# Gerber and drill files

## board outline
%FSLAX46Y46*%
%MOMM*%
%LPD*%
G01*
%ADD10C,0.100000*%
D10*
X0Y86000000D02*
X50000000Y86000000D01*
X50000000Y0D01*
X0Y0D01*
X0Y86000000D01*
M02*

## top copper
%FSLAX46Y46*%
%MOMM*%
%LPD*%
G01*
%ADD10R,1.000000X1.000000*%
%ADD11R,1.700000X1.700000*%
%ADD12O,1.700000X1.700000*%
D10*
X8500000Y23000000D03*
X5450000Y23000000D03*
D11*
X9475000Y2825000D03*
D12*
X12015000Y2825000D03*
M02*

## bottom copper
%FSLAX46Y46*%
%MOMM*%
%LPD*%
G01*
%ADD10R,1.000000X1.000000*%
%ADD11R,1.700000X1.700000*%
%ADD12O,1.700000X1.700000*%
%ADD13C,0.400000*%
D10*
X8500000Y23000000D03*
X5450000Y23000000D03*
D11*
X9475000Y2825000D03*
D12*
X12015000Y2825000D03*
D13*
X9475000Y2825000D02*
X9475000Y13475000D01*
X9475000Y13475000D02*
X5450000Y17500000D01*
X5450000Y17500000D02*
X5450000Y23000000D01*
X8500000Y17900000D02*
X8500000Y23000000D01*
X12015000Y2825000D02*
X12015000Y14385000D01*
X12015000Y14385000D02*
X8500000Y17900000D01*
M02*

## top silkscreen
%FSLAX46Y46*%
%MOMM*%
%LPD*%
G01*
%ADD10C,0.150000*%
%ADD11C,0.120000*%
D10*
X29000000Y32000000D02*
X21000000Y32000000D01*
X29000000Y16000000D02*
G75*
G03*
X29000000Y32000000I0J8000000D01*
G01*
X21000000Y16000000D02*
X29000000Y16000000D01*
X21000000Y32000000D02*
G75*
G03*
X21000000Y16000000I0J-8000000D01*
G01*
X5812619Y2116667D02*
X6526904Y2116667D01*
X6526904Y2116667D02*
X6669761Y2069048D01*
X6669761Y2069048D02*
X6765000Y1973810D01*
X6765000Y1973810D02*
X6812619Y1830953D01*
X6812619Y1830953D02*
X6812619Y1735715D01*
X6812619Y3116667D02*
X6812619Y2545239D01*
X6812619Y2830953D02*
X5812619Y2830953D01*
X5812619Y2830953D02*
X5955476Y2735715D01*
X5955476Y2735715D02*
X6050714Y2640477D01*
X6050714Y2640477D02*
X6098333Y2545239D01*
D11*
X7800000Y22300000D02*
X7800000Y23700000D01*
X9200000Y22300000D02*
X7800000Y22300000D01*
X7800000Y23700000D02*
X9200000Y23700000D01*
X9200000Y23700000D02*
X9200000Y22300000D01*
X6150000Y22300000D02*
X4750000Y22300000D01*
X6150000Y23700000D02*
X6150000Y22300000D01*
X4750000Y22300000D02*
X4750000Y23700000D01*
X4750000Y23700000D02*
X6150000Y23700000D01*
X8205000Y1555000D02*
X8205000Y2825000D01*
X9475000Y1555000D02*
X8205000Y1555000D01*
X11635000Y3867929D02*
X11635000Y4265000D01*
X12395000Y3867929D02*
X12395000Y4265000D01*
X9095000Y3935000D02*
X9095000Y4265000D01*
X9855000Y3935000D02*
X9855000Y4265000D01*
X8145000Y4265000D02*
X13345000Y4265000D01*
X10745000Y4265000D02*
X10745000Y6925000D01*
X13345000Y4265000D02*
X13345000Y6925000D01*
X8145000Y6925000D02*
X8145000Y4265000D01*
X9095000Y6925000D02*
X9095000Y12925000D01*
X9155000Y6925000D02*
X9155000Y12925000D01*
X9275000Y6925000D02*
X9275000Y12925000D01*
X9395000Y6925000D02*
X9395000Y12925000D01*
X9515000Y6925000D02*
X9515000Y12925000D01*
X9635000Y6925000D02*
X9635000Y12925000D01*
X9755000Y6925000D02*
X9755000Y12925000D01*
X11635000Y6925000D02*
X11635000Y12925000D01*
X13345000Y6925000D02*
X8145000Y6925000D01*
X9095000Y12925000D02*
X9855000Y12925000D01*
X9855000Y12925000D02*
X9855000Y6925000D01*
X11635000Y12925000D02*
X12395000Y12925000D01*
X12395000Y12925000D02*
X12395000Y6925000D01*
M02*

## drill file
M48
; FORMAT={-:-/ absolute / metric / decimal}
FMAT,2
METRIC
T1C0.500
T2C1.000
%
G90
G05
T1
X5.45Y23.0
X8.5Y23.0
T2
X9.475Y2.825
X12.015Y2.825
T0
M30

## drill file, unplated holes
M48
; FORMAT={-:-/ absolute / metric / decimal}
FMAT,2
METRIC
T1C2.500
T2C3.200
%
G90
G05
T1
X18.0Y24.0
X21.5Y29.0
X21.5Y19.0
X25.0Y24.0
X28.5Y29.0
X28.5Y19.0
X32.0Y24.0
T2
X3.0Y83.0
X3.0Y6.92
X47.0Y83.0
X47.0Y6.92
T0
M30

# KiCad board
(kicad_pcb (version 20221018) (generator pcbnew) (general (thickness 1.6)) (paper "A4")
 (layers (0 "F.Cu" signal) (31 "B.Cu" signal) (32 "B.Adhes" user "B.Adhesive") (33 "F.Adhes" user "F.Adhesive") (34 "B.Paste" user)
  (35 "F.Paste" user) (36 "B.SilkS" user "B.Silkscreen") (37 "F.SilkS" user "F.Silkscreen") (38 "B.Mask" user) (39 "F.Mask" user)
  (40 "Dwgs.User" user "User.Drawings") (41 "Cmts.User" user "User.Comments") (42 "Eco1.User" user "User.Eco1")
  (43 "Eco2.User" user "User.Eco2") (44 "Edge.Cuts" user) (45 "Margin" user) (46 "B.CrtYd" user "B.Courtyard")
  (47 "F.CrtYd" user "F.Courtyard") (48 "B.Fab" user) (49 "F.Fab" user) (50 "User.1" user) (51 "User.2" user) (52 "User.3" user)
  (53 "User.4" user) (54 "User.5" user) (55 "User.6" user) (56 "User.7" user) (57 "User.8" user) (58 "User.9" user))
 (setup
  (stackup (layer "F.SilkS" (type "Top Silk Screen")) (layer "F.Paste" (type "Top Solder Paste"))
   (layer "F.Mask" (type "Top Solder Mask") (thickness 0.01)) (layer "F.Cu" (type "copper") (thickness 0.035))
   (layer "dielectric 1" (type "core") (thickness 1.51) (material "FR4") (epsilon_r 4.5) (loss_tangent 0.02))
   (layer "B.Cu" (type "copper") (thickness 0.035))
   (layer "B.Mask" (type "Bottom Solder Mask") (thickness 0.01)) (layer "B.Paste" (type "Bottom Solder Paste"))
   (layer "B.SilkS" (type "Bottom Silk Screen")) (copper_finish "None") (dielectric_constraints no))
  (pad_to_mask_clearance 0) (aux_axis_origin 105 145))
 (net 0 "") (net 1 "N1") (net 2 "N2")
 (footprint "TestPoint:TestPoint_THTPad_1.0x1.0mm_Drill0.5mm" (layer "F.Cu") (at 113.5 122 90)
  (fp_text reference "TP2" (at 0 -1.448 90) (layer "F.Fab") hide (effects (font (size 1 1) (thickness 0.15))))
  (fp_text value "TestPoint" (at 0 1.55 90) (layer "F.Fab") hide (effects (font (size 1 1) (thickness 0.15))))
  (fp_line (start -0.7 -0.7) (end 0.7 -0.7) (stroke (width 0.12) (type solid)) (layer "F.SilkS"))
  (fp_line (start -0.7 0.7) (end -0.7 -0.7) (stroke (width 0.12) (type solid)) (layer "F.SilkS"))
  (fp_line (start 0.7 -0.7) (end 0.7 0.7) (stroke (width 0.12) (type solid)) (layer "F.SilkS"))
  (fp_line (start 0.7 0.7) (end -0.7 0.7) (stroke (width 0.12) (type solid)) (layer "F.SilkS"))
  (pad "1" thru_hole rect (at 0 0 90) (size 1 1) (drill 0.5) (layers "*.Cu" "*.Mask") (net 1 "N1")))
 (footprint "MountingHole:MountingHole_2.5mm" (layer "F.Cu") (at 133.5 116)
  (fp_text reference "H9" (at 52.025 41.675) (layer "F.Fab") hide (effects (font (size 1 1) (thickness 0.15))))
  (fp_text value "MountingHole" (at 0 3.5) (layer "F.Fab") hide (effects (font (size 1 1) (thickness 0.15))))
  (pad "" np_thru_hole circle (at 0 0) (size 2.5 2.5) (drill 2.5) (layers "*.Cu" "*.Mask")))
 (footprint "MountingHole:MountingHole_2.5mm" (layer "F.Cu") (at 137 121)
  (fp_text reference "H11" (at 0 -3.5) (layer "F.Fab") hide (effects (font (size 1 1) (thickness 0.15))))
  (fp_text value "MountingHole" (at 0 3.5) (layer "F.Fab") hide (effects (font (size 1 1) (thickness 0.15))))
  (pad "" np_thru_hole circle (at 0 0) (size 2.5 2.5) (drill 2.5) (layers "*.Cu" "*.Mask")))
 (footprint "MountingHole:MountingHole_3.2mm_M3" (layer "F.Cu") (at 108 138.08)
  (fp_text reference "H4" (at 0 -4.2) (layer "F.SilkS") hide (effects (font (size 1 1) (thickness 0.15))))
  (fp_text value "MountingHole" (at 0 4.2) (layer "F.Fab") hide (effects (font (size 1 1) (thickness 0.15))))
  (pad "" np_thru_hole circle (at 0 0) (size 3.2 3.2) (drill 3.2) (layers "F&B.Cu" "*.Mask") (clearance 1.6)))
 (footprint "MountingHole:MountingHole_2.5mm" (layer "F.Cu") (at 126.5 126)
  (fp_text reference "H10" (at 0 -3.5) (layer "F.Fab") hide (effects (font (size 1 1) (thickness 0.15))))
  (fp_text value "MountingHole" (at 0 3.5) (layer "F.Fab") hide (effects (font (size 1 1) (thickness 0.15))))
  (pad "" np_thru_hole circle (at 0 0) (size 2.5 2.5) (drill 2.5) (layers "*.Cu" "*.Mask")))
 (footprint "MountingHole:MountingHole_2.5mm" (layer "F.Cu") (at 133.5 126)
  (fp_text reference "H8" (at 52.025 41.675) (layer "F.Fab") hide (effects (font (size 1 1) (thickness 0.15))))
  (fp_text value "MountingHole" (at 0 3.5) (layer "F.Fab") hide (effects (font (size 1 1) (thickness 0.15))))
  (pad "" np_thru_hole circle (at 0 0) (size 2.5 2.5) (drill 2.5) (layers "*.Cu" "*.Mask")))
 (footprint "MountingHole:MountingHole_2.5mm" (layer "F.Cu") (at 130 121)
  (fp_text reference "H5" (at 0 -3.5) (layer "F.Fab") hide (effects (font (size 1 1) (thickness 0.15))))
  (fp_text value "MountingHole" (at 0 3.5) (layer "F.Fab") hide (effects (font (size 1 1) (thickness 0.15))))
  (pad "" np_thru_hole circle (at 0 0) (size 2.5 2.5) (drill 2.5) (layers "*.Cu" "*.Mask")))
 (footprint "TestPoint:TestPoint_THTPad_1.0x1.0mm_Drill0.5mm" (layer "F.Cu") (at 110.45 122 180)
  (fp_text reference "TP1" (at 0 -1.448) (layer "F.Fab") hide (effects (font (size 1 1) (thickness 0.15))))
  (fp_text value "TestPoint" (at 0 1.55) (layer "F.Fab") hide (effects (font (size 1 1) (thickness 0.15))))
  (fp_line (start -0.7 -0.7) (end 0.7 -0.7) (stroke (width 0.12) (type solid)) (layer "F.SilkS"))
  (fp_line (start -0.7 0.7) (end -0.7 -0.7) (stroke (width 0.12) (type solid)) (layer "F.SilkS"))
  (fp_line (start 0.7 -0.7) (end 0.7 0.7) (stroke (width 0.12) (type solid)) (layer "F.SilkS"))
  (fp_line (start 0.7 0.7) (end -0.7 0.7) (stroke (width 0.12) (type solid)) (layer "F.SilkS"))
  (pad "1" thru_hole rect (at 0 0 180) (size 1 1) (drill 0.5) (layers "*.Cu" "*.Mask") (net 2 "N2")))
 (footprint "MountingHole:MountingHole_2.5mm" (layer "F.Cu") (at 126.5 116)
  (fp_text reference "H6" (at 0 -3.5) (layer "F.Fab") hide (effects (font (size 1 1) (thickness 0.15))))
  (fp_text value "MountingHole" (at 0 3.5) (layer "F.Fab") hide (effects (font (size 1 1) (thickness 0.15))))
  (pad "" np_thru_hole circle (at 0 0) (size 2.5 2.5) (drill 2.5) (layers "*.Cu" "*.Mask")))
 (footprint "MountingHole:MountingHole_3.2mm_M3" (layer "F.Cu") (at 152 62)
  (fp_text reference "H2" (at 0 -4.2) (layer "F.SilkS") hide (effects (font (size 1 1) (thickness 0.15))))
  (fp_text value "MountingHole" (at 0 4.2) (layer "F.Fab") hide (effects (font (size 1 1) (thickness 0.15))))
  (pad "" np_thru_hole circle (at 0 0) (size 3.2 3.2) (drill 3.2) (layers "*.Cu" "*.Mask")))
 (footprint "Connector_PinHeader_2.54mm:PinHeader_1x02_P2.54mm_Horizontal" (layer "F.Cu") (at 114.475 142.175 90)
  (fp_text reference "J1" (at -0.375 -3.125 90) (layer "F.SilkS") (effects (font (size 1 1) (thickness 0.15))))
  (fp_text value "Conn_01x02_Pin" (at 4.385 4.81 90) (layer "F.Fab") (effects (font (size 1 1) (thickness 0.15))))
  (fp_line (start -1.27 -1.27) (end 0 -1.27) (stroke (width 0.12) (type solid)) (layer "F.SilkS"))
  (fp_line (start -1.27 0) (end -1.27 -1.27) (stroke (width 0.12) (type solid)) (layer "F.SilkS"))
  (fp_line (start 1.042929 2.16) (end 1.44 2.16) (stroke (width 0.12) (type solid)) (layer "F.SilkS"))
  (fp_line (start 1.042929 2.92) (end 1.44 2.92) (stroke (width 0.12) (type solid)) (layer "F.SilkS"))
  (fp_line (start 1.11 -0.38) (end 1.44 -0.38) (stroke (width 0.12) (type solid)) (layer "F.SilkS"))
  (fp_line (start 1.11 0.38) (end 1.44 0.38) (stroke (width 0.12) (type solid)) (layer "F.SilkS"))
  (fp_line (start 1.44 -1.33) (end 1.44 3.87) (stroke (width 0.12) (type solid)) (layer "F.SilkS"))
  (fp_line (start 1.44 1.27) (end 4.1 1.27) (stroke (width 0.12) (type solid)) (layer "F.SilkS"))
  (fp_line (start 1.44 3.87) (end 4.1 3.87) (stroke (width 0.12) (type solid)) (layer "F.SilkS"))
  (fp_line (start 4.1 -1.33) (end 1.44 -1.33) (stroke (width 0.12) (type solid)) (layer "F.SilkS"))
  (fp_line (start 4.1 -0.38) (end 10.1 -0.38) (stroke (width 0.12) (type solid)) (layer "F.SilkS"))
  (fp_line (start 4.1 -0.32) (end 10.1 -0.32) (stroke (width 0.12) (type solid)) (layer "F.SilkS"))
  (fp_line (start 4.1 -0.2) (end 10.1 -0.2) (stroke (width 0.12) (type solid)) (layer "F.SilkS"))
  (fp_line (start 4.1 -0.08) (end 10.1 -0.08) (stroke (width 0.12) (type solid)) (layer "F.SilkS"))
  (fp_line (start 4.1 0.04) (end 10.1 0.04) (stroke (width 0.12) (type solid)) (layer "F.SilkS"))
  (fp_line (start 4.1 0.16) (end 10.1 0.16) (stroke (width 0.12) (type solid)) (layer "F.SilkS"))
  (fp_line (start 4.1 0.28) (end 10.1 0.28) (stroke (width 0.12) (type solid)) (layer "F.SilkS"))
  (fp_line (start 4.1 2.16) (end 10.1 2.16) (stroke (width 0.12) (type solid)) (layer "F.SilkS"))
  (fp_line (start 4.1 3.87) (end 4.1 -1.33) (stroke (width 0.12) (type solid)) (layer "F.SilkS"))
  (fp_line (start 10.1 -0.38) (end 10.1 0.38) (stroke (width 0.12) (type solid)) (layer "F.SilkS"))
  (fp_line (start 10.1 0.38) (end 4.1 0.38) (stroke (width 0.12) (type solid)) (layer "F.SilkS"))
  (fp_line (start 10.1 2.16) (end 10.1 2.92) (stroke (width 0.12) (type solid)) (layer "F.SilkS"))
  (fp_line (start 10.1 2.92) (end 4.1 2.92) (stroke (width 0.12) (type solid)) (layer "F.SilkS"))
  (pad "1" thru_hole rect (at 0 0 90) (size 1.7 1.7) (drill 1) (layers "*.Cu" "*.Mask") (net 2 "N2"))
  (pad "2" thru_hole oval (at 0 2.54 90) (size 1.7 1.7) (drill 1) (layers "*.Cu" "*.Mask") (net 1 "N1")))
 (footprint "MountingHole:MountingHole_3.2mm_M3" (layer "F.Cu") (at 108 62)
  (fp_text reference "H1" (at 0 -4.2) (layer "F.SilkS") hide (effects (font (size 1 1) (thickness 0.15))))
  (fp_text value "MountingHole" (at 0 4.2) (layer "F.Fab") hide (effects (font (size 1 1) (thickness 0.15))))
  (pad "" np_thru_hole circle (at 0 0) (size 3.2 3.2) (drill 3.2) (layers "*.Cu" "*.Mask")))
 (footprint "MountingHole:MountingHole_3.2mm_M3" (layer "F.Cu") (at 152 138.08)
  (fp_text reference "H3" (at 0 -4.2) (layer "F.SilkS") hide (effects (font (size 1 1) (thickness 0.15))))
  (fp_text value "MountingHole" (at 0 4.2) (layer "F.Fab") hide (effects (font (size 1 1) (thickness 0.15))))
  (pad "" np_thru_hole circle (at 0 0) (size 3.2 3.2) (drill 3.2) (layers "*.Cu" "*.Mask")))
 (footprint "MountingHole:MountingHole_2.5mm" (layer "F.Cu") (at 123 121)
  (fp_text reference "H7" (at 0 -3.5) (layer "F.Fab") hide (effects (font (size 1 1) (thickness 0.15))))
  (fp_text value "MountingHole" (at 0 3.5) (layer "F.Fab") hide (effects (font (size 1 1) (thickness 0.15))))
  (pad "" np_thru_hole circle (at 0 0) (size 2.5 2.5) (drill 2.5) (layers "*.Cu" "*.Mask")))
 (gr_line (start 134 113) (end 126 113) (stroke (width 0.15) (type default)) (layer "F.SilkS"))
 (gr_arc (start 134 113) (mid 142 121) (end 134 129) (stroke (width 0.15) (type default)) (layer "F.SilkS"))
 (gr_line (start 126 129) (end 134 129) (stroke (width 0.15) (type default)) (layer "F.SilkS"))
 (gr_arc (start 126 129) (mid 118 121) (end 126 113) (stroke (width 0.15) (type default)) (layer "F.SilkS"))
 (gr_rect (start 105 59) (end 155 145) (stroke (width 0.1) (type default)) (fill none) (layer "Edge.Cuts"))
 (segment (start 114.475 142.175) (end 114.475 131.525) (width 0.4) (layer "B.Cu") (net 2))
 (segment (start 114.475 131.525) (end 110.45 127.5) (width 0.4) (layer "B.Cu") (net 2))
 (segment (start 110.45 127.5) (end 110.45 122) (width 0.4) (layer "B.Cu") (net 2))
 (segment (start 113.5 127.1) (end 113.5 122) (width 0.4) (layer "B.Cu") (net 1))
 (segment (start 117.015 142.175) (end 117.015 130.615) (width 0.4) (layer "B.Cu") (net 1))
 (segment (start 117.015 130.615) (end 113.5 127.1) (width 0.4) (layer "B.Cu") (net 1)))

